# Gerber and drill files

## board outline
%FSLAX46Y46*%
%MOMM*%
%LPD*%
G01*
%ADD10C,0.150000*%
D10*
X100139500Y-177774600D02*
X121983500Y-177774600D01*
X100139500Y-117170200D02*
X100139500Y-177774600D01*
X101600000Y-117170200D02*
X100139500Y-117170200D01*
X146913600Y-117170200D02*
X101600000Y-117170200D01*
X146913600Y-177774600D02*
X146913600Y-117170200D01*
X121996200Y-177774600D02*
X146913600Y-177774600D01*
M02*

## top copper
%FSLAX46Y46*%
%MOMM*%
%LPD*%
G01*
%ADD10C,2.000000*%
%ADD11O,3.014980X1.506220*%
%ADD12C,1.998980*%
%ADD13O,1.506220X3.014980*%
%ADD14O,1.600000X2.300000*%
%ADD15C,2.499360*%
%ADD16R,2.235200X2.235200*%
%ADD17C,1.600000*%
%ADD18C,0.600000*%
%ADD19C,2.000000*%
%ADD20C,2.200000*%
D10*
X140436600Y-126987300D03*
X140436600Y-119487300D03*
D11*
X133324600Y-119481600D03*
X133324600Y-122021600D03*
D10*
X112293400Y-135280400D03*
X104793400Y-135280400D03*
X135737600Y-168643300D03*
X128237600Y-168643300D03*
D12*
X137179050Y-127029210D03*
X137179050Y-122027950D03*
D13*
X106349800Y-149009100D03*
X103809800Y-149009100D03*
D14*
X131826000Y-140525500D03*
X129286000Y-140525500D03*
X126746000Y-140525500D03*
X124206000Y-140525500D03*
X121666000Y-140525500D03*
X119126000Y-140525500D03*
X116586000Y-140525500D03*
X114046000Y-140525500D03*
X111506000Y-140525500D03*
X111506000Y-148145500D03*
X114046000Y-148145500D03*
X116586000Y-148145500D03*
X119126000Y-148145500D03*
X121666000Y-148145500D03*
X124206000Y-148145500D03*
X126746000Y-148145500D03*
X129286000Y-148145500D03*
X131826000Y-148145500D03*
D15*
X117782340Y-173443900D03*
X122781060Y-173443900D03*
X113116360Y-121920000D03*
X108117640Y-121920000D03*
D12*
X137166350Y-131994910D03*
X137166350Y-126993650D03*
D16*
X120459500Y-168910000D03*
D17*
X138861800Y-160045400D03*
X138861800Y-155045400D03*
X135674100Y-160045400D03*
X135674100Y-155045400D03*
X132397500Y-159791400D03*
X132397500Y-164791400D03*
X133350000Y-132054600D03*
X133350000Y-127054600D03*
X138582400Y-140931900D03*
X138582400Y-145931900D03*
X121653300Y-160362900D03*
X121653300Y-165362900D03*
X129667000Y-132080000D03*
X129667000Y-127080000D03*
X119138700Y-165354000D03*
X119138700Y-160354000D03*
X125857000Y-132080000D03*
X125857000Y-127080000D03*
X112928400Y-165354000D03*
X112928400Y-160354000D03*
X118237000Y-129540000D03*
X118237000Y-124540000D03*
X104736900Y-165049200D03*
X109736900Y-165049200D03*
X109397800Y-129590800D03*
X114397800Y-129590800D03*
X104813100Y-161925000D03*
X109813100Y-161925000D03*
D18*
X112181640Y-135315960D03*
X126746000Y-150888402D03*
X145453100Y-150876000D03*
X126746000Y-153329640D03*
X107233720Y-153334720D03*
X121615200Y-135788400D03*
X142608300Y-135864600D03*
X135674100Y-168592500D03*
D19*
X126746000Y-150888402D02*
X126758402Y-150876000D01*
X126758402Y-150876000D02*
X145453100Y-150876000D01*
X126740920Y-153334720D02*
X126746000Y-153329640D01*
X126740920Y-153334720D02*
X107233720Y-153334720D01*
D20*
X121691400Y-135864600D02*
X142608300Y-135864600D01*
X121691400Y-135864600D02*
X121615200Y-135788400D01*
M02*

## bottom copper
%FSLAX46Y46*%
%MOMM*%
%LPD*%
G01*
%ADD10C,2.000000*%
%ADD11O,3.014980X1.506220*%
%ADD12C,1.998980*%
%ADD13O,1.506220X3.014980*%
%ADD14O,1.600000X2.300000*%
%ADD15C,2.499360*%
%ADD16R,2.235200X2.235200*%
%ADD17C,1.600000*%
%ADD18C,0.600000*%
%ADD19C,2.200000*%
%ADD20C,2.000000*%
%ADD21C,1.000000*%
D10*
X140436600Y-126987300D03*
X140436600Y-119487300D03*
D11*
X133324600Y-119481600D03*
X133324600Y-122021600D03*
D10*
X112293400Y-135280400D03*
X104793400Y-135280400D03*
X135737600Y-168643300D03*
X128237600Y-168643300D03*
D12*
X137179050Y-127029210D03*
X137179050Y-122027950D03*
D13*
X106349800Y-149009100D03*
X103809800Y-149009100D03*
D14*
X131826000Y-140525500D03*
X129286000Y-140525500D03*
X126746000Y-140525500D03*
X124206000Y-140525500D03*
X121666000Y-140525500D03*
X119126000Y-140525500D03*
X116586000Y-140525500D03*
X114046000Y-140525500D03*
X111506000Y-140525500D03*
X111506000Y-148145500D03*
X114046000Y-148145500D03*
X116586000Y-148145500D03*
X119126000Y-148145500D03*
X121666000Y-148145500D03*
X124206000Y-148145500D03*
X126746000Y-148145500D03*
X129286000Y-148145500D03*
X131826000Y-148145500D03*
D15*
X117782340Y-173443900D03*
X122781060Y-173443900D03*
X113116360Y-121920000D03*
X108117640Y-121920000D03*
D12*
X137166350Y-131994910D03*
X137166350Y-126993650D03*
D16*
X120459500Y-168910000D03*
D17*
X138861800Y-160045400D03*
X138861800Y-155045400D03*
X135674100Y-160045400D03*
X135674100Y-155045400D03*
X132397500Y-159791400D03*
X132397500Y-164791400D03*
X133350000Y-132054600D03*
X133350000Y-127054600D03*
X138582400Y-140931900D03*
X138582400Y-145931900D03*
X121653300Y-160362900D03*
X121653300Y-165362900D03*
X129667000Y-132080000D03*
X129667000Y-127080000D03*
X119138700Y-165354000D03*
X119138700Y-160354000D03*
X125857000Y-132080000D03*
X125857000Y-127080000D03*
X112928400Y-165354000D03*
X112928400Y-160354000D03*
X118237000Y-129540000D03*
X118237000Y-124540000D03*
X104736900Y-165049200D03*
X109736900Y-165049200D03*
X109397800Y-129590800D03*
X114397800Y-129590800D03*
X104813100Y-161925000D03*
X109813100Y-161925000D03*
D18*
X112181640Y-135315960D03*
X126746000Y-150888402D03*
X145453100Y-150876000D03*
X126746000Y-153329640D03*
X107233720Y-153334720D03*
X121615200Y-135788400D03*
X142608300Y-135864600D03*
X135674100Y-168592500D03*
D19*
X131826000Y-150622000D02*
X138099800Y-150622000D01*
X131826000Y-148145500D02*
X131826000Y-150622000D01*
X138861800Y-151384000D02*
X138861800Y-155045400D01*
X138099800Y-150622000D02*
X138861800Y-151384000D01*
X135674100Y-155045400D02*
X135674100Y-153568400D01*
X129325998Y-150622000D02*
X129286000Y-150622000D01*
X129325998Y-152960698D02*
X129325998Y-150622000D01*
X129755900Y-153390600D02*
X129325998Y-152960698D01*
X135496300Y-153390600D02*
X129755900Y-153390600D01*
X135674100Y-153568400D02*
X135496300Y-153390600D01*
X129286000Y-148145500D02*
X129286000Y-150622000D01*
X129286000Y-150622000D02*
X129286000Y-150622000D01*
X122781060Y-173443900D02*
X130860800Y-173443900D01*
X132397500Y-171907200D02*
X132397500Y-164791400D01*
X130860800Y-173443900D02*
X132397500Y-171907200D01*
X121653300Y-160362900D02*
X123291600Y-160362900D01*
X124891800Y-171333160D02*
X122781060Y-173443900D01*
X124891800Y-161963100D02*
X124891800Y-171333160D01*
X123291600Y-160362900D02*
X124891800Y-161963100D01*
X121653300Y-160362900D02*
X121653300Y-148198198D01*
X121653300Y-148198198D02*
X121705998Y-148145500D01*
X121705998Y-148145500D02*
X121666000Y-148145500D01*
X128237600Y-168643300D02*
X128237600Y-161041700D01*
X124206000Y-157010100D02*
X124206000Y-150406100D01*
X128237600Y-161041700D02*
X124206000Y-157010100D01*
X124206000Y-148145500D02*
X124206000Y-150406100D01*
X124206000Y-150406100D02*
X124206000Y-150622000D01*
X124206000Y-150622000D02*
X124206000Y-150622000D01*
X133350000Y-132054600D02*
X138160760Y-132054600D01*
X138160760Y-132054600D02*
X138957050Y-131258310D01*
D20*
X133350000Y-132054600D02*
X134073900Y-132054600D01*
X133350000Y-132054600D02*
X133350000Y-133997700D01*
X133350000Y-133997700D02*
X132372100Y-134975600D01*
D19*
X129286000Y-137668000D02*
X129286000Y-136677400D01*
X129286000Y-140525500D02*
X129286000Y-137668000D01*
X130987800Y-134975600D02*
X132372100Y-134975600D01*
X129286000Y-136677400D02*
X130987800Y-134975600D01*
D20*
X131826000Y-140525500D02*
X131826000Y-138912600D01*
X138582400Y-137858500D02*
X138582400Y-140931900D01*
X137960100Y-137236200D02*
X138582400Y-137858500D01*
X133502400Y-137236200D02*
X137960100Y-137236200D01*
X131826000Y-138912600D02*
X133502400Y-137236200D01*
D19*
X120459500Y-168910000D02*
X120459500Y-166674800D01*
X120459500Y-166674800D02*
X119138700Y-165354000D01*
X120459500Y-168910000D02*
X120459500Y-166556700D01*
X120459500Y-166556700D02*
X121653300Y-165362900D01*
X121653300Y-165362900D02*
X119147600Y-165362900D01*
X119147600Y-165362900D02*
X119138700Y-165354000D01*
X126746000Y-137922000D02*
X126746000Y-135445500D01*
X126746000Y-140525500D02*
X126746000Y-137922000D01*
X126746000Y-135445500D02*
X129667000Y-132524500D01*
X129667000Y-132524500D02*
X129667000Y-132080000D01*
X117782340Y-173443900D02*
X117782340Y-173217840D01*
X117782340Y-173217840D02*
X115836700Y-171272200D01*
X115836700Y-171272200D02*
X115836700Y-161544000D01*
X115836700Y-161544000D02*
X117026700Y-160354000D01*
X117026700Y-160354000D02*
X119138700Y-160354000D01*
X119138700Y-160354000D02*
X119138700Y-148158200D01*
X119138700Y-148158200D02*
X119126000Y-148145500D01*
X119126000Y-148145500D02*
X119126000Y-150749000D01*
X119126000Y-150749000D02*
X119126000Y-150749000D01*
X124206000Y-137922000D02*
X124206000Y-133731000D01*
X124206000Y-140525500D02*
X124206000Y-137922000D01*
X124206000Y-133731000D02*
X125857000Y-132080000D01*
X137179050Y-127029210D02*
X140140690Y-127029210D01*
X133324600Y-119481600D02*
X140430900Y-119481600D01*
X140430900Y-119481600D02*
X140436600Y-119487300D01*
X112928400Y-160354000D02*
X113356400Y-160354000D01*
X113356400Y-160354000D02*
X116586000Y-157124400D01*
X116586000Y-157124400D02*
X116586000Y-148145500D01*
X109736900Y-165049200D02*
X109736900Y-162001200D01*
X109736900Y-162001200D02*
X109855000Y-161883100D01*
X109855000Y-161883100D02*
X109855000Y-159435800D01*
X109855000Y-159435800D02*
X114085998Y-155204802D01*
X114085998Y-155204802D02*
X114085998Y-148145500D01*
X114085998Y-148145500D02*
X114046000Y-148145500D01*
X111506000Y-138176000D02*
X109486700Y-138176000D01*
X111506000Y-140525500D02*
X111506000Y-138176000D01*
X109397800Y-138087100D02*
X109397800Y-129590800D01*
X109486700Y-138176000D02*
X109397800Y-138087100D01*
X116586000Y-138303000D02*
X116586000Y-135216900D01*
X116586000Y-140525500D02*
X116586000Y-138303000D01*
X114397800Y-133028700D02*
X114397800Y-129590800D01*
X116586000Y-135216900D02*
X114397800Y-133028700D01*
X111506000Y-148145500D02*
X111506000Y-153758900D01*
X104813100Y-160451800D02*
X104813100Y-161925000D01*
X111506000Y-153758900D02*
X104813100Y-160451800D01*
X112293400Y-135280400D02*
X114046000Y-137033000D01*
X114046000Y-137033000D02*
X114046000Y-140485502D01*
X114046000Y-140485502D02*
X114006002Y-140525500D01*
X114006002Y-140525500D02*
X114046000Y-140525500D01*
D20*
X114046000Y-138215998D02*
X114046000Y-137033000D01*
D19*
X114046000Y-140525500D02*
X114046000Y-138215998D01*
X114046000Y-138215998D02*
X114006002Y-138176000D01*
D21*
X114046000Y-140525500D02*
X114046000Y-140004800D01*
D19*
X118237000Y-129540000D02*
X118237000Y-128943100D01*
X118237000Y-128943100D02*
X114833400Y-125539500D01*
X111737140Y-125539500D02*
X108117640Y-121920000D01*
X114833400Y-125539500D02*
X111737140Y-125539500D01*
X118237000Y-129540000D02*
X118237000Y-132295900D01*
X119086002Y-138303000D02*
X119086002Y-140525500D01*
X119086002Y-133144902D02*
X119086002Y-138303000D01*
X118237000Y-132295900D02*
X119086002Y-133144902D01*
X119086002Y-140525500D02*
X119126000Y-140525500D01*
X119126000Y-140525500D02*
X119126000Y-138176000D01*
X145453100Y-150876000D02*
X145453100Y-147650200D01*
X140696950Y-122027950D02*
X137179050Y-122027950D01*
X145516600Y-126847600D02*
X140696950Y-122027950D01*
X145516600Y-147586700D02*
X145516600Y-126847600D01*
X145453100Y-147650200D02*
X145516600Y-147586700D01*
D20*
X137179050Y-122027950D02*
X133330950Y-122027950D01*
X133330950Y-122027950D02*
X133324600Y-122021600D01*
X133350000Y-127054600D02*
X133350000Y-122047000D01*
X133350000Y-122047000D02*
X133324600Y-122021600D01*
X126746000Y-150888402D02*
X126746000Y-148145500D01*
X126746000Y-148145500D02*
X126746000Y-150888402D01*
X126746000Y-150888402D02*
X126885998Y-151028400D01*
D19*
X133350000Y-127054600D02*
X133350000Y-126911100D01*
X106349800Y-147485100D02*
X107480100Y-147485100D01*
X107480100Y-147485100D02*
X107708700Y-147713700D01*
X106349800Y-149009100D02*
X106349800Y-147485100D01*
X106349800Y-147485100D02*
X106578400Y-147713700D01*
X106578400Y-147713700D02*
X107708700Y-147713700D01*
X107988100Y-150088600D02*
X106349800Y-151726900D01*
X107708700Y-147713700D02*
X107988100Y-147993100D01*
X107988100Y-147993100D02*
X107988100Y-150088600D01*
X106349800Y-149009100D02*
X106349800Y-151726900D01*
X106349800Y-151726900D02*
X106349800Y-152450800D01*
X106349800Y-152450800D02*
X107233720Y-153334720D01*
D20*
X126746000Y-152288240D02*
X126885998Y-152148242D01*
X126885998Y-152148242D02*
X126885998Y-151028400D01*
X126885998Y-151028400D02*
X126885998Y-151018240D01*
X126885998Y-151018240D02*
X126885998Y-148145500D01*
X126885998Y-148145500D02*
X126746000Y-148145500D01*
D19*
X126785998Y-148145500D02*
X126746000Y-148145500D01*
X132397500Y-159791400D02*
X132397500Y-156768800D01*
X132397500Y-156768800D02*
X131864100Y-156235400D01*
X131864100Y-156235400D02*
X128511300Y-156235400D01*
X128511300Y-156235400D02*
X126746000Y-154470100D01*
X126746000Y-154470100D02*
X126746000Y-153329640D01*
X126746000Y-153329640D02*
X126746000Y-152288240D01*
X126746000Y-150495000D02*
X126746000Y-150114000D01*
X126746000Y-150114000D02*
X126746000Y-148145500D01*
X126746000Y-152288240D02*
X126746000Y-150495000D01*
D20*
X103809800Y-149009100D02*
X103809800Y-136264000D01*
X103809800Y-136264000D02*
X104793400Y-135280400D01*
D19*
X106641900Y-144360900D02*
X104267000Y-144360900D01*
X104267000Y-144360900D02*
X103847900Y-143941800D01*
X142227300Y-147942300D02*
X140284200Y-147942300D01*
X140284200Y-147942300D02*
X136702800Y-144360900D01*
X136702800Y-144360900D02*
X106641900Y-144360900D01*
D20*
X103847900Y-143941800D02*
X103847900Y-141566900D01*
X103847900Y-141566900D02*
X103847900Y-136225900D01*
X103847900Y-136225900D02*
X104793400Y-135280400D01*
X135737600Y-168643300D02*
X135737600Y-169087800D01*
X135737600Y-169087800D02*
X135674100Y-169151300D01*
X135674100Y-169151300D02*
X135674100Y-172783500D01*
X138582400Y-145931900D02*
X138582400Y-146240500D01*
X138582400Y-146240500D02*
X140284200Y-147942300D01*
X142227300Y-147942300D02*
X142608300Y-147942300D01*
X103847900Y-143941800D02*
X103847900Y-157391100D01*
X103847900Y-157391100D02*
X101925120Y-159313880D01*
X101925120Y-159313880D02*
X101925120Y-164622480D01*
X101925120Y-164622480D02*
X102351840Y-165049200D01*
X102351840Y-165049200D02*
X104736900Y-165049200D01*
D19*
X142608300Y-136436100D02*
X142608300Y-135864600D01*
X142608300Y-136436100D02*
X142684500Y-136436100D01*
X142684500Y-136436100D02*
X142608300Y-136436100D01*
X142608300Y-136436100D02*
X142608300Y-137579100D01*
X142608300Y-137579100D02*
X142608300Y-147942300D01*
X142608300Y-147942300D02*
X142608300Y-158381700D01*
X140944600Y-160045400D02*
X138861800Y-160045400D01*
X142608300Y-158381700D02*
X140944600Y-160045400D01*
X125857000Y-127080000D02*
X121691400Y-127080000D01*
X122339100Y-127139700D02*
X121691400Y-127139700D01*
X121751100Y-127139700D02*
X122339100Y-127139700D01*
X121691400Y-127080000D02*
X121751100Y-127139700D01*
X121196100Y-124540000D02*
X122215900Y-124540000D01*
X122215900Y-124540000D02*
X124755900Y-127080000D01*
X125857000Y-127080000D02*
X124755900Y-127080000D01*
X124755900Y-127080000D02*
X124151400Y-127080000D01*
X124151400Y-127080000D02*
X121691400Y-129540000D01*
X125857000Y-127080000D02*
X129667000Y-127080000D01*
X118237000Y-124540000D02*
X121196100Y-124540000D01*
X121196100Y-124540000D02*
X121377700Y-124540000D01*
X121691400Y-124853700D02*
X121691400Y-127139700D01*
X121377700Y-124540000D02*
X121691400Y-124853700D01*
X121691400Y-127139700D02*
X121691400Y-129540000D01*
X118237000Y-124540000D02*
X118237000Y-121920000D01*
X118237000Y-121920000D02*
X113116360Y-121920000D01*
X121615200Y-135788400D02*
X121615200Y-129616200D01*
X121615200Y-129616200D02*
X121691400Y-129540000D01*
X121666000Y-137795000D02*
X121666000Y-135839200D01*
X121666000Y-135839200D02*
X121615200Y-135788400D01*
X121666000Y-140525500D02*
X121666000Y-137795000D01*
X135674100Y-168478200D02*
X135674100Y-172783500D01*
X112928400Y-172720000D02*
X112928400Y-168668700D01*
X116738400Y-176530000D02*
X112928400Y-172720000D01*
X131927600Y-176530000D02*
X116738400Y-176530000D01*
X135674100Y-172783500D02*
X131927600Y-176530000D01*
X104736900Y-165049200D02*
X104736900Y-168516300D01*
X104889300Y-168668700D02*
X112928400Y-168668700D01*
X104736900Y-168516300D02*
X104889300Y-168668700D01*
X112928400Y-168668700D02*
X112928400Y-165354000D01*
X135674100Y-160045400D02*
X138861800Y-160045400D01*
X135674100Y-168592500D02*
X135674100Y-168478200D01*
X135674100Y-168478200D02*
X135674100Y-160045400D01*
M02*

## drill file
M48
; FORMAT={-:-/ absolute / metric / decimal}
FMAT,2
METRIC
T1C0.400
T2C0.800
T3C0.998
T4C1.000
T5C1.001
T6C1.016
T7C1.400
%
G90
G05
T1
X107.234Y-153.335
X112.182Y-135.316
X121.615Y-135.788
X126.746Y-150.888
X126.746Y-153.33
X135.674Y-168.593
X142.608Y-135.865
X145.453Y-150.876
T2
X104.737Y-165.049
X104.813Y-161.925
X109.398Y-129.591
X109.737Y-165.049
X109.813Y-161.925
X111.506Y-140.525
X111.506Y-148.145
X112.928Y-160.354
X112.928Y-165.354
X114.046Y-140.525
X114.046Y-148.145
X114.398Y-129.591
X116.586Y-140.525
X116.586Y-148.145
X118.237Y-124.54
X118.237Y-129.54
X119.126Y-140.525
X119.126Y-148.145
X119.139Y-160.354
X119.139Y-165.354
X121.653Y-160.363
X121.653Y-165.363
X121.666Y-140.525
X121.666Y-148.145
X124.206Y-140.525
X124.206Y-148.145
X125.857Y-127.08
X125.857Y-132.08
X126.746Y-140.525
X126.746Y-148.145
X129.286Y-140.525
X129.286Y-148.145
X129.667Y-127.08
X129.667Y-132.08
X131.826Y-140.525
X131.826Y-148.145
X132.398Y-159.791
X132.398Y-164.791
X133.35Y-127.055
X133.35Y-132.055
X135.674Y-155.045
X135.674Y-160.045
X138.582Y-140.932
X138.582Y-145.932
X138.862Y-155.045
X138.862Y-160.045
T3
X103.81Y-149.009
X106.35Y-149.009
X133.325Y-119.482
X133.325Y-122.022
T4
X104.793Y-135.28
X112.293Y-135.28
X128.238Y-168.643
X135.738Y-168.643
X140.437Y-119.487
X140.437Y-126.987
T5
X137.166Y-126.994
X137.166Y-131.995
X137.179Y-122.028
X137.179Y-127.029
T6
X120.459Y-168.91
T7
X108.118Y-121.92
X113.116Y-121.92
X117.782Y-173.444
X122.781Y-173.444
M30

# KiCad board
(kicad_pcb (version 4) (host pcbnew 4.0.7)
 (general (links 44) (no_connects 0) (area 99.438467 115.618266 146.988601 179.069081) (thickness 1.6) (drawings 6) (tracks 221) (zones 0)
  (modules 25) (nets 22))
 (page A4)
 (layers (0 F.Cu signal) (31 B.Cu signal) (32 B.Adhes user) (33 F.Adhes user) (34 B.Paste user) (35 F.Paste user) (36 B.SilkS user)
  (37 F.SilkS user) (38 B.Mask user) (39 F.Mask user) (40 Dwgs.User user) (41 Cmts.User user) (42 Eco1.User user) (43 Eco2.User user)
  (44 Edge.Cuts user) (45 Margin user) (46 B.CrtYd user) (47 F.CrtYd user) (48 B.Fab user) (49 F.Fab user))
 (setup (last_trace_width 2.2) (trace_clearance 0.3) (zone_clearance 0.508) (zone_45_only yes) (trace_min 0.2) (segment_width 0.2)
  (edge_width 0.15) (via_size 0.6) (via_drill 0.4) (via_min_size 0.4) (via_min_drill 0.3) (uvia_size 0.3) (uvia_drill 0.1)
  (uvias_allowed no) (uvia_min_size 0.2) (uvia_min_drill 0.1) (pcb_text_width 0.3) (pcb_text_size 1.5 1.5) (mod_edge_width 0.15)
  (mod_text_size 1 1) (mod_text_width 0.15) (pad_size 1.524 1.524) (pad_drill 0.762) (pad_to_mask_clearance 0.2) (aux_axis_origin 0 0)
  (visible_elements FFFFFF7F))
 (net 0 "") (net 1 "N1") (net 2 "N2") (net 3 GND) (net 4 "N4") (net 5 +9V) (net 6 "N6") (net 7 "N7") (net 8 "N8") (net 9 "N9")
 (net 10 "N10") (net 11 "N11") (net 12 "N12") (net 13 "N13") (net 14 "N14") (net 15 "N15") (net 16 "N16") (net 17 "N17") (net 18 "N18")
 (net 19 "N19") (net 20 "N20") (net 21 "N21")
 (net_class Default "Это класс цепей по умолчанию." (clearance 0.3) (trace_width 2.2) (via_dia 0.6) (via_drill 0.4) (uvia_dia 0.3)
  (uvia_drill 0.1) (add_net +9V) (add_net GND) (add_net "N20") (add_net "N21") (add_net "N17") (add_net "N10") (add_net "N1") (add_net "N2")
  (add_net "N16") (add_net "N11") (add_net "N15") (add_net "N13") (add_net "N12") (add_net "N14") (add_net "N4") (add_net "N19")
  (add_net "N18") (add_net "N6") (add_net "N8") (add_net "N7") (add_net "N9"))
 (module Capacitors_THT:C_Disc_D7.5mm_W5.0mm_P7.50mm (layer F.Cu) (at 140.4366 126.9873 90)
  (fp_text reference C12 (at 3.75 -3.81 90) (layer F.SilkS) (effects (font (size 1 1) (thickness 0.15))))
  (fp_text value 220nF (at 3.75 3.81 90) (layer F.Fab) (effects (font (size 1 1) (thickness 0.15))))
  (pad 1 thru_hole circle (at 0 0 90) (size 2 2) (drill 1) (layers *.Cu *.Mask) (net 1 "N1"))
  (pad 2 thru_hole circle (at 7.5 0 90) (size 2 2) (drill 1) (layers *.Cu *.Mask) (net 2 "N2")))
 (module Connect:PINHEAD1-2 (layer F.Cu) (at 133.3246 120.7516 270)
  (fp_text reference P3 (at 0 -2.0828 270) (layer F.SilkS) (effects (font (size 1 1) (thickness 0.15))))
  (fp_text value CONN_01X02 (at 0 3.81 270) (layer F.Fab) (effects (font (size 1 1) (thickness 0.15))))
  (pad 1 thru_hole oval (at -1.27 0 270) (size 1.50622 3.01498) (drill 0.99822) (layers *.Cu *.Mask) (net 2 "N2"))
  (pad 2 thru_hole oval (at 1.27 0 270) (size 1.50622 3.01498) (drill 0.99822) (layers *.Cu *.Mask) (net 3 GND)))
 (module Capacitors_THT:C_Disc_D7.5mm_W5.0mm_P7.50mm (layer F.Cu) (at 112.2934 135.2804 180)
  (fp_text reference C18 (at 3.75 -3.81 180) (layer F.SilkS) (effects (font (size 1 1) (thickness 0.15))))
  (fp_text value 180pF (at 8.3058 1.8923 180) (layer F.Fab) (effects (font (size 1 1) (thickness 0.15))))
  (pad 1 thru_hole circle (at 0 0 180) (size 2 2) (drill 1) (layers *.Cu *.Mask) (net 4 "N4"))
  (pad 2 thru_hole circle (at 7.5 0 180) (size 2 2) (drill 1) (layers *.Cu *.Mask) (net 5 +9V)))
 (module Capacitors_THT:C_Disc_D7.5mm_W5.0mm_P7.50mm (layer F.Cu) (at 135.7376 168.6433 180)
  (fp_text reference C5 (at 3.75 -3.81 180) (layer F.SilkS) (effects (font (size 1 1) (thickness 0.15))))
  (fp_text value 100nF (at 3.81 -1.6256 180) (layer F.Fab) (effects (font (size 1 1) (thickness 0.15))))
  (pad 1 thru_hole circle (at 0 0 180) (size 2 2) (drill 1) (layers *.Cu *.Mask) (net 5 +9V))
  (pad 2 thru_hole circle (at 7.5 0 180) (size 2 2) (drill 1) (layers *.Cu *.Mask) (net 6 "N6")))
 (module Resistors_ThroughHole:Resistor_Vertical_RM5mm (layer F.Cu) (at 137.17905 124.52985 90)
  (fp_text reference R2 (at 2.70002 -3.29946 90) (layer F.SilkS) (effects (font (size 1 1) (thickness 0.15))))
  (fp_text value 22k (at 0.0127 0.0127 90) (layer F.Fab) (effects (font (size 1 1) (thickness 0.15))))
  (pad 1 thru_hole circle (at -2.49936 0 90) (size 1.99898 1.99898) (drill 1.00076) (layers *.Cu *.SilkS *.Mask) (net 1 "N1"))
  (pad 2 thru_hole circle (at 2.5019 0 90) (size 1.99898 1.99898) (drill 1.00076) (layers *.Cu *.SilkS *.Mask) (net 3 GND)))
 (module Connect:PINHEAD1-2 (layer F.Cu) (at 105.0798 149.0091 180)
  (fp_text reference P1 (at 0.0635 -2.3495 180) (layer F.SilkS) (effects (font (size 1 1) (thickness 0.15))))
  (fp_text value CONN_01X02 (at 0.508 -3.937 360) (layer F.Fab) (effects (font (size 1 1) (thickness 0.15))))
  (pad 1 thru_hole oval (at -1.27 0 180) (size 1.50622 3.01498) (drill 0.99822) (layers *.Cu *.Mask) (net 3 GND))
  (pad 2 thru_hole oval (at 1.27 0 180) (size 1.50622 3.01498) (drill 0.99822) (layers *.Cu *.Mask) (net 5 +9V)))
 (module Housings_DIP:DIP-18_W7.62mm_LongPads (layer F.Cu) (at 131.826 140.5255 270)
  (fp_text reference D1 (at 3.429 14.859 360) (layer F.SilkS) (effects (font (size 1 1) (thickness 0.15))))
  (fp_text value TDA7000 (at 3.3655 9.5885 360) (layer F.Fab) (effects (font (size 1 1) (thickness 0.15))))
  (pad 1 thru_hole oval (at 0 0 270) (size 2.3 1.6) (drill 0.8) (layers *.Cu *.Mask F.SilkS) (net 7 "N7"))
  (pad 2 thru_hole oval (at 0 2.54 270) (size 2.3 1.6) (drill 0.8) (layers *.Cu *.Mask F.SilkS) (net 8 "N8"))
  (pad 3 thru_hole oval (at 0 5.08 270) (size 2.3 1.6) (drill 0.8) (layers *.Cu *.Mask F.SilkS) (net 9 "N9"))
  (pad 4 thru_hole oval (at 0 7.62 270) (size 2.3 1.6) (drill 0.8) (layers *.Cu *.Mask F.SilkS) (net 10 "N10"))
  (pad 5 thru_hole oval (at 0 10.16 270) (size 2.3 1.6) (drill 0.8) (layers *.Cu *.Mask F.SilkS) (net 5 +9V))
  (pad 6 thru_hole oval (at 0 12.7 270) (size 2.3 1.6) (drill 0.8) (layers *.Cu *.Mask F.SilkS) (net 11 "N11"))
  (pad 7 thru_hole oval (at 0 15.24 270) (size 2.3 1.6) (drill 0.8) (layers *.Cu *.Mask F.SilkS) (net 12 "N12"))
  (pad 8 thru_hole oval (at 0 17.78 270) (size 2.3 1.6) (drill 0.8) (layers *.Cu *.Mask F.SilkS) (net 4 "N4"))
  (pad 9 thru_hole oval (at 0 20.32 270) (size 2.3 1.6) (drill 0.8) (layers *.Cu *.Mask F.SilkS) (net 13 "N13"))
  (pad 10 thru_hole oval (at 7.62 20.32 270) (size 2.3 1.6) (drill 0.8) (layers *.Cu *.Mask F.SilkS) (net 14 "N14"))
  (pad 11 thru_hole oval (at 7.62 17.78 270) (size 2.3 1.6) (drill 0.8) (layers *.Cu *.Mask F.SilkS) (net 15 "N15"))
  (pad 12 thru_hole oval (at 7.62 15.24 270) (size 2.3 1.6) (drill 0.8) (layers *.Cu *.Mask F.SilkS) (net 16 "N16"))
  (pad 13 thru_hole oval (at 7.62 12.7 270) (size 2.3 1.6) (drill 0.8) (layers *.Cu *.Mask F.SilkS) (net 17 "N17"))
  (pad 14 thru_hole oval (at 7.62 10.16 270) (size 2.3 1.6) (drill 0.8) (layers *.Cu *.Mask F.SilkS) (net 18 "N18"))
  (pad 15 thru_hole oval (at 7.62 7.62 270) (size 2.3 1.6) (drill 0.8) (layers *.Cu *.Mask F.SilkS) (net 6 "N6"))
  (pad 16 thru_hole oval (at 7.62 5.08 270) (size 2.3 1.6) (drill 0.8) (layers *.Cu *.Mask F.SilkS) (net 3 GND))
  (pad 17 thru_hole oval (at 7.62 2.54 270) (size 2.3 1.6) (drill 0.8) (layers *.Cu *.Mask F.SilkS) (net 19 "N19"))
  (pad 18 thru_hole oval (at 7.62 0 270) (size 2.3 1.6) (drill 0.8) (layers *.Cu *.Mask F.SilkS) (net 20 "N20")))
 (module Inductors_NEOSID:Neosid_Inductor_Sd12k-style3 (layer F.Cu) (at 120.2817 173.4439 180)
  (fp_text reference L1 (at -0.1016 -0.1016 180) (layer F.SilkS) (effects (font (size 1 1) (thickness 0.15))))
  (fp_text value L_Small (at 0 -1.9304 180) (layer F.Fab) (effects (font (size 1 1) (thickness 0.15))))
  (pad 2 thru_hole circle (at 2.49936 0 180) (size 2.49936 2.49936) (drill 1.39954) (layers *.Cu *.Mask F.SilkS) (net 17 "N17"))
  (pad 1 thru_hole circle (at -2.49936 0 180) (size 2.49936 2.49936) (drill 1.39954) (layers *.Cu *.Mask F.SilkS) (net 18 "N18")))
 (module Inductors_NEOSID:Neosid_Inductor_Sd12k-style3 (layer F.Cu) (at 110.617 121.92)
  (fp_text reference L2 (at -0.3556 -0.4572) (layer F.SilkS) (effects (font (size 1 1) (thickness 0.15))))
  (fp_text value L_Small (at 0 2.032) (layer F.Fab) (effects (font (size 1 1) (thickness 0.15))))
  (pad 2 thru_hole circle (at 2.49936 0) (size 2.49936 2.49936) (drill 1.39954) (layers *.Cu *.Mask F.SilkS) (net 5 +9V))
  (pad 1 thru_hole circle (at -2.49936 0) (size 2.49936 2.49936) (drill 1.39954) (layers *.Cu *.Mask F.SilkS) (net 11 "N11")))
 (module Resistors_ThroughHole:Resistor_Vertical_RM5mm (layer F.Cu) (at 137.16635 129.49555 90)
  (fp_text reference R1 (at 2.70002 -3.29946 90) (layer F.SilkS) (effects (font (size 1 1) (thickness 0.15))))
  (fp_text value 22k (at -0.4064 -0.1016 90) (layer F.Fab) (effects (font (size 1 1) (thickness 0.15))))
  (pad 1 thru_hole circle (at -2.49936 0 90) (size 1.99898 1.99898) (drill 1.00076) (layers *.Cu *.SilkS *.Mask) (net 8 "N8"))
  (pad 2 thru_hole circle (at 2.5019 0 90) (size 1.99898 1.99898) (drill 1.00076) (layers *.Cu *.SilkS *.Mask) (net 1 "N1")))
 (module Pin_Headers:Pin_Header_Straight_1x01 (layer F.Cu) (at 120.4595 168.91)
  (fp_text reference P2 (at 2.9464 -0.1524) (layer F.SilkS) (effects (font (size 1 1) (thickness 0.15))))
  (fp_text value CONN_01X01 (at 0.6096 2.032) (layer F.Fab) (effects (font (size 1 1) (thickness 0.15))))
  (pad 1 thru_hole rect (at 0 0) (size 2.2352 2.2352) (drill 1.016) (layers *.Cu *.Mask F.SilkS) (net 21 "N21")))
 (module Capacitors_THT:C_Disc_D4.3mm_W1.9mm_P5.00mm (layer F.Cu) (at 138.8618 160.0454 90)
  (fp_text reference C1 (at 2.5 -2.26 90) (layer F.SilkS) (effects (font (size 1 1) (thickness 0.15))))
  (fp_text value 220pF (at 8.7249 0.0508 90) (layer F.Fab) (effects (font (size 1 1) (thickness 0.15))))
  (pad 1 thru_hole circle (at 0 0 90) (size 1.6 1.6) (drill 0.8) (layers *.Cu *.Mask) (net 5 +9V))
  (pad 2 thru_hole circle (at 5 0 90) (size 1.6 1.6) (drill 0.8) (layers *.Cu *.Mask) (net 20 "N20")))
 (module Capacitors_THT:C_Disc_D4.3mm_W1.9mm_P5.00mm (layer F.Cu) (at 135.6741 160.0454 90)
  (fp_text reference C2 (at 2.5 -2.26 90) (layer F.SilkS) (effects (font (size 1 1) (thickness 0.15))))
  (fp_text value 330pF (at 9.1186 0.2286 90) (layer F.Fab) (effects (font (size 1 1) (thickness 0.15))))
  (pad 1 thru_hole circle (at 0 0 90) (size 1.6 1.6) (drill 0.8) (layers *.Cu *.Mask) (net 5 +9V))
  (pad 2 thru_hole circle (at 5 0 90) (size 1.6 1.6) (drill 0.8) (layers *.Cu *.Mask) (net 19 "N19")))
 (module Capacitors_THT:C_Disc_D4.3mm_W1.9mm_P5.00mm (layer F.Cu) (at 132.3975 159.7914 270)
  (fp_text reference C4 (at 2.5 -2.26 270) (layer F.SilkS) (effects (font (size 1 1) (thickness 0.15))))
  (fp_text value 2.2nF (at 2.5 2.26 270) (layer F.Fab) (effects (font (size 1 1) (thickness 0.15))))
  (pad 1 thru_hole circle (at 0 0 270) (size 1.6 1.6) (drill 0.8) (layers *.Cu *.Mask) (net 3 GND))
  (pad 2 thru_hole circle (at 5 0 270) (size 1.6 1.6) (drill 0.8) (layers *.Cu *.Mask) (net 18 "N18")))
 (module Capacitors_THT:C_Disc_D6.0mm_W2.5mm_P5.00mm (layer F.Cu) (at 133.35 132.0546 90)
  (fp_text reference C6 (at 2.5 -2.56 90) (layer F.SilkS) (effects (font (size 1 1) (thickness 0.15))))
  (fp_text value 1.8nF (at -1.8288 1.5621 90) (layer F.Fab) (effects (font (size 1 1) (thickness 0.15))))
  (pad 1 thru_hole circle (at 0 0 90) (size 1.6 1.6) (drill 0.8) (layers *.Cu *.Mask) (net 8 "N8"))
  (pad 2 thru_hole circle (at 5 0 90) (size 1.6 1.6) (drill 0.8) (layers *.Cu *.Mask) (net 3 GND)))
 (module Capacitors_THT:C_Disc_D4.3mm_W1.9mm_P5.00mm (layer F.Cu) (at 138.5824 140.9319 270)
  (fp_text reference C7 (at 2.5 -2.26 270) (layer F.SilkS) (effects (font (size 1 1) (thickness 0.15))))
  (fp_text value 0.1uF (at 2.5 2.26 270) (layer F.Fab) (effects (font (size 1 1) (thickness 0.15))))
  (pad 1 thru_hole circle (at 0 0 270) (size 1.6 1.6) (drill 0.8) (layers *.Cu *.Mask) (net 7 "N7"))
  (pad 2 thru_hole circle (at 5 0 270) (size 1.6 1.6) (drill 0.8) (layers *.Cu *.Mask) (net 5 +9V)))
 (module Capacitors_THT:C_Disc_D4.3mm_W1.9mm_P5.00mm (layer F.Cu) (at 121.6533 160.3629 270)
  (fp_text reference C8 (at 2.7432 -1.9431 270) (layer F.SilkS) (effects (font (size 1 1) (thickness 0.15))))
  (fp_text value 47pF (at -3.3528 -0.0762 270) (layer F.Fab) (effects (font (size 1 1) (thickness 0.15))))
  (pad 1 thru_hole circle (at 0 0 270) (size 1.6 1.6) (drill 0.8) (layers *.Cu *.Mask) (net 18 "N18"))
  (pad 2 thru_hole circle (at 5 0 270) (size 1.6 1.6) (drill 0.8) (layers *.Cu *.Mask) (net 21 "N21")))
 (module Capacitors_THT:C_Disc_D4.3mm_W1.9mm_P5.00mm (layer F.Cu) (at 129.667 132.08 90)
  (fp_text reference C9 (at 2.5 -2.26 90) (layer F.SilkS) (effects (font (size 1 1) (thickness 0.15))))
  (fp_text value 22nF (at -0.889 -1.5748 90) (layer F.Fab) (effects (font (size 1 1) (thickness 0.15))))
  (pad 1 thru_hole circle (at 0 0 90) (size 1.6 1.6) (drill 0.8) (layers *.Cu *.Mask) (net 9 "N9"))
  (pad 2 thru_hole circle (at 5 0 90) (size 1.6 1.6) (drill 0.8) (layers *.Cu *.Mask) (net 5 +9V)))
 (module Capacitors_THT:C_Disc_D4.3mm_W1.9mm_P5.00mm (layer F.Cu) (at 119.1387 165.354 90)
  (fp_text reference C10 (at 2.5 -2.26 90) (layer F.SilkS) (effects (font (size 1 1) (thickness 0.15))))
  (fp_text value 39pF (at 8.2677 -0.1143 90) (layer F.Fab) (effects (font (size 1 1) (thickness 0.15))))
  (pad 1 thru_hole circle (at 0 0 90) (size 1.6 1.6) (drill 0.8) (layers *.Cu *.Mask) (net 21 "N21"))
  (pad 2 thru_hole circle (at 5 0 90) (size 1.6 1.6) (drill 0.8) (layers *.Cu *.Mask) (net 17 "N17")))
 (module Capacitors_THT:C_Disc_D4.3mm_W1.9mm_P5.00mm (layer F.Cu) (at 125.857 132.08 90)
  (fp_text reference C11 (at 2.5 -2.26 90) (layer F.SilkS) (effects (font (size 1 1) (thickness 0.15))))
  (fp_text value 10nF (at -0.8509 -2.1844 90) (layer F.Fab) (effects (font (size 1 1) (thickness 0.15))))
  (pad 1 thru_hole circle (at 0 0 90) (size 1.6 1.6) (drill 0.8) (layers *.Cu *.Mask) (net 10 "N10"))
  (pad 2 thru_hole circle (at 5 0 90) (size 1.6 1.6) (drill 0.8) (layers *.Cu *.Mask) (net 5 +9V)))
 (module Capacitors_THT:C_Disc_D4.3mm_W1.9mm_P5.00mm (layer F.Cu) (at 112.9284 165.354 90)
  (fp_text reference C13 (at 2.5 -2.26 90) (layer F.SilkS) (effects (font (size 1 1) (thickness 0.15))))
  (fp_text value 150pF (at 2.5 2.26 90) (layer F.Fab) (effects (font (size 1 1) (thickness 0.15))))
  (pad 1 thru_hole circle (at 0 0 90) (size 1.6 1.6) (drill 0.8) (layers *.Cu *.Mask) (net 5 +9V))
  (pad 2 thru_hole circle (at 5 0 90) (size 1.6 1.6) (drill 0.8) (layers *.Cu *.Mask) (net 16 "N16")))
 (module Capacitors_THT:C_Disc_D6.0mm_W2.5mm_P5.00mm (layer F.Cu) (at 118.237 129.54 90)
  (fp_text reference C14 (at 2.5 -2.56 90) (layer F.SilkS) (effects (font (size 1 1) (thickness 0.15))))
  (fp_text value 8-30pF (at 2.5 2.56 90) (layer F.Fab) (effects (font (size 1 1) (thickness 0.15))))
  (pad 1 thru_hole circle (at 0 0 90) (size 1.6 1.6) (drill 0.8) (layers *.Cu *.Mask) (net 11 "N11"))
  (pad 2 thru_hole circle (at 5 0 90) (size 1.6 1.6) (drill 0.8) (layers *.Cu *.Mask) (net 5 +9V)))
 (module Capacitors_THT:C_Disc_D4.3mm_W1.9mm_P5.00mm (layer F.Cu) (at 104.7369 165.0492)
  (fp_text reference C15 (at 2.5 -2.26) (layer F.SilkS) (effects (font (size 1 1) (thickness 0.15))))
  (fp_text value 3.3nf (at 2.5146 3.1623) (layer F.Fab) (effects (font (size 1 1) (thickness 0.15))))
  (pad 1 thru_hole circle (at 0 0) (size 1.6 1.6) (drill 0.8) (layers *.Cu *.Mask) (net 5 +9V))
  (pad 2 thru_hole circle (at 5 0) (size 1.6 1.6) (drill 0.8) (layers *.Cu *.Mask) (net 15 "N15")))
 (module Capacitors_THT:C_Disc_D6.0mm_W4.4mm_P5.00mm (layer F.Cu) (at 109.3978 129.5908)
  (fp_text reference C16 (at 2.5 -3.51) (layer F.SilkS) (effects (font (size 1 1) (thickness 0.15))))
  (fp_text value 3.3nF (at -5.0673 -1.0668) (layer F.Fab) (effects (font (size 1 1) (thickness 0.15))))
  (pad 1 thru_hole circle (at 0 0) (size 1.6 1.6) (drill 0.8) (layers *.Cu *.Mask) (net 13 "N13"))
  (pad 2 thru_hole circle (at 5 0) (size 1.6 1.6) (drill 0.8) (layers *.Cu *.Mask) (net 12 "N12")))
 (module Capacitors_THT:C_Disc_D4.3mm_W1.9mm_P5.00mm (layer F.Cu) (at 104.8131 161.925)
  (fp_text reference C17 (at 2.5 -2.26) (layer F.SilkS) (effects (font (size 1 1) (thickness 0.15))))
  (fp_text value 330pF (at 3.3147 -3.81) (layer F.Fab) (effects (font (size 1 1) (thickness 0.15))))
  (pad 1 thru_hole circle (at 0 0) (size 1.6 1.6) (drill 0.8) (layers *.Cu *.Mask) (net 14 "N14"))
  (pad 2 thru_hole circle (at 5 0) (size 1.6 1.6) (drill 0.8) (layers *.Cu *.Mask) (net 15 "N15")))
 (gr_line (start 100.1395 177.7746) (end 121.9835 177.7746) (angle 90) (layer Edge.Cuts) (width 0.15))
 (gr_line (start 100.1395 117.1702) (end 100.1395 177.7746) (angle 90) (layer Edge.Cuts) (width 0.15))
 (gr_line (start 101.6 117.1702) (end 100.1395 117.1702) (angle 90) (layer Edge.Cuts) (width 0.15))
 (gr_line (start 146.9136 117.1702) (end 101.6 117.1702) (angle 90) (layer Edge.Cuts) (width 0.15))
 (gr_line (start 146.9136 177.7746) (end 146.9136 117.1702) (angle 90) (layer Edge.Cuts) (width 0.15))
 (gr_line (start 121.9962 177.7746) (end 146.9136 177.7746) (angle 90) (layer Edge.Cuts) (width 0.15))
 (segment (start 131.826 150.622) (end 138.0998 150.622) (width 2.2) (layer B.Cu) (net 20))
 (segment (start 131.826 148.1455) (end 131.826 150.622) (width 2.2) (layer B.Cu) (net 20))
 (segment (start 138.8618 151.384) (end 138.8618 155.0454) (width 2.2) (layer B.Cu) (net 20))
 (segment (start 138.0998 150.622) (end 138.8618 151.384) (width 2.2) (layer B.Cu) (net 20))
 (segment (start 135.6741 155.0454) (end 135.6741 153.5684) (width 2.2) (layer B.Cu) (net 19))
 (segment (start 129.325998 150.622) (end 129.286 150.622) (width 2.2) (layer B.Cu) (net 19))
 (segment (start 129.325998 152.960698) (end 129.325998 150.622) (width 2.2) (layer B.Cu) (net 19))
 (segment (start 129.7559 153.3906) (end 129.325998 152.960698) (width 2.2) (layer B.Cu) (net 19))
 (segment (start 135.4963 153.3906) (end 129.7559 153.3906) (width 2.2) (layer B.Cu) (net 19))
 (segment (start 135.6741 153.5684) (end 135.4963 153.3906) (width 2.2) (layer B.Cu) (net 19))
 (segment (start 129.286 148.1455) (end 129.286 150.622) (width 2.2) (layer B.Cu) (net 19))
 (segment (start 129.286 150.622) (end 129.286 150.622) (width 2.2) (layer B.Cu) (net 19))
 (segment (start 122.78106 173.4439) (end 130.8608 173.4439) (width 2.2) (layer B.Cu) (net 18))
 (segment (start 132.3975 171.9072) (end 132.3975 164.7914) (width 2.2) (layer B.Cu) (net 18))
 (segment (start 130.8608 173.4439) (end 132.3975 171.9072) (width 2.2) (layer B.Cu) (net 18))
 (segment (start 121.6533 160.3629) (end 123.2916 160.3629) (width 2.2) (layer B.Cu) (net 18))
 (segment (start 124.8918 171.33316) (end 122.78106 173.4439) (width 2.2) (layer B.Cu) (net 18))
 (segment (start 124.8918 161.9631) (end 124.8918 171.33316) (width 2.2) (layer B.Cu) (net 18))
 (segment (start 123.2916 160.3629) (end 124.8918 161.9631) (width 2.2) (layer B.Cu) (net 18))
 (segment (start 121.6533 160.3629) (end 121.6533 148.198198) (width 2.2) (layer B.Cu) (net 18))
 (segment (start 121.6533 148.198198) (end 121.705998 148.1455) (width 2.2) (layer B.Cu) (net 18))
 (segment (start 121.705998 148.1455) (end 121.666 148.1455) (width 2.2) (layer B.Cu) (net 18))
 (segment (start 128.2376 168.6433) (end 128.2376 161.0417) (width 2.2) (layer B.Cu) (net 6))
 (segment (start 124.206 157.0101) (end 124.206 150.4061) (width 2.2) (layer B.Cu) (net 6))
 (segment (start 128.2376 161.0417) (end 124.206 157.0101) (width 2.2) (layer B.Cu) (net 6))
 (segment (start 124.206 148.1455) (end 124.206 150.4061) (width 2.2) (layer B.Cu) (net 6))
 (segment (start 124.206 150.4061) (end 124.206 150.622) (width 2.2) (layer B.Cu) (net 6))
 (segment (start 124.206 150.622) (end 124.206 150.622) (width 2.2) (layer B.Cu) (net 6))
 (segment (start 133.35 132.0546) (end 138.16076 132.0546) (width 2.2) (layer B.Cu) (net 8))
 (segment (start 138.16076 132.0546) (end 138.95705 131.25831) (width 2.2) (layer B.Cu) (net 8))
 (segment (start 133.35 132.0546) (end 134.0739 132.0546) (width 2) (layer B.Cu) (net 8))
 (segment (start 133.35 132.0546) (end 133.35 133.9977) (width 2) (layer B.Cu) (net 8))
 (segment (start 133.35 133.9977) (end 132.3721 134.9756) (width 2) (layer B.Cu) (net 8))
 (segment (start 129.286 137.668) (end 129.286 136.6774) (width 2.2) (layer B.Cu) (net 8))
 (segment (start 129.286 140.5255) (end 129.286 137.668) (width 2.2) (layer B.Cu) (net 8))
 (segment (start 130.9878 134.9756) (end 132.3721 134.9756) (width 2.2) (layer B.Cu) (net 8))
 (segment (start 129.286 136.6774) (end 130.9878 134.9756) (width 2.2) (layer B.Cu) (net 8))
 (segment (start 131.826 140.5255) (end 131.826 138.9126) (width 2) (layer B.Cu) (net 7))
 (segment (start 138.5824 137.8585) (end 138.5824 140.9319) (width 2) (layer B.Cu) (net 7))
 (segment (start 137.9601 137.2362) (end 138.5824 137.8585) (width 2) (layer B.Cu) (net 7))
 (segment (start 133.5024 137.2362) (end 137.9601 137.2362) (width 2) (layer B.Cu) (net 7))
 (segment (start 131.826 138.9126) (end 133.5024 137.2362) (width 2) (layer B.Cu) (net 7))
 (segment (start 120.4595 168.91) (end 120.4595 166.6748) (width 2.2) (layer B.Cu) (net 21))
 (segment (start 120.4595 166.6748) (end 119.1387 165.354) (width 2.2) (layer B.Cu) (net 21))
 (segment (start 120.4595 168.91) (end 120.4595 166.5567) (width 2.2) (layer B.Cu) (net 21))
 (segment (start 120.4595 166.5567) (end 121.6533 165.3629) (width 2.2) (layer B.Cu) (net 21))
 (segment (start 121.6533 165.3629) (end 119.1476 165.3629) (width 2.2) (layer B.Cu) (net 21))
 (segment (start 119.1476 165.3629) (end 119.1387 165.354) (width 2.2) (layer B.Cu) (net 21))
 (segment (start 126.746 137.922) (end 126.746 135.4455) (width 2.2) (layer B.Cu) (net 9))
 (segment (start 126.746 140.5255) (end 126.746 137.922) (width 2.2) (layer B.Cu) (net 9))
 (segment (start 126.746 135.4455) (end 129.667 132.5245) (width 2.2) (layer B.Cu) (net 9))
 (segment (start 129.667 132.5245) (end 129.667 132.08) (width 2.2) (layer B.Cu) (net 9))
 (segment (start 117.78234 173.4439) (end 117.78234 173.21784) (width 2.2) (layer B.Cu) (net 17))
 (segment (start 117.78234 173.21784) (end 115.8367 171.2722) (width 2.2) (layer B.Cu) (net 17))
 (segment (start 115.8367 171.2722) (end 115.8367 161.544) (width 2.2) (layer B.Cu) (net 17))
 (segment (start 115.8367 161.544) (end 117.0267 160.354) (width 2.2) (layer B.Cu) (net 17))
 (segment (start 117.0267 160.354) (end 119.1387 160.354) (width 2.2) (layer B.Cu) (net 17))
 (segment (start 119.1387 160.354) (end 119.1387 148.1582) (width 2.2) (layer B.Cu) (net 17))
 (segment (start 119.1387 148.1582) (end 119.126 148.1455) (width 2.2) (layer B.Cu) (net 17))
 (segment (start 119.126 148.1455) (end 119.126 150.749) (width 2.2) (layer B.Cu) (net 17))
 (segment (start 119.126 150.749) (end 119.126 150.749) (width 2.2) (layer B.Cu) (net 17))
 (segment (start 124.206 137.922) (end 124.206 133.731) (width 2.2) (layer B.Cu) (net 10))
 (segment (start 124.206 140.5255) (end 124.206 137.922) (width 2.2) (layer B.Cu) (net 10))
 (segment (start 124.206 133.731) (end 125.857 132.08) (width 2.2) (layer B.Cu) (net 10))
 (segment (start 137.17905 127.02921) (end 140.14069 127.02921) (width 2.2) (layer B.Cu) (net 1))
 (segment (start 133.3246 119.4816) (end 140.4309 119.4816) (width 2.2) (layer B.Cu) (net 2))
 (segment (start 140.4309 119.4816) (end 140.4366 119.4873) (width 2.2) (layer B.Cu) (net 2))
 (segment (start 112.9284 160.354) (end 113.3564 160.354) (width 2.2) (layer B.Cu) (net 16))
 (segment (start 113.3564 160.354) (end 116.586 157.1244) (width 2.2) (layer B.Cu) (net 16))
 (segment (start 116.586 157.1244) (end 116.586 148.1455) (width 2.2) (layer B.Cu) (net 16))
 (segment (start 109.7369 165.0492) (end 109.7369 162.0012) (width 2.2) (layer B.Cu) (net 15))
 (segment (start 109.7369 162.0012) (end 109.855 161.8831) (width 2.2) (layer B.Cu) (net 15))
 (segment (start 109.855 161.8831) (end 109.855 159.4358) (width 2.2) (layer B.Cu) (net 15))
 (segment (start 109.855 159.4358) (end 114.085998 155.204802) (width 2.2) (layer B.Cu) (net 15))
 (segment (start 114.085998 155.204802) (end 114.085998 148.1455) (width 2.2) (layer B.Cu) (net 15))
 (segment (start 114.085998 148.1455) (end 114.046 148.1455) (width 2.2) (layer B.Cu) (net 15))
 (segment (start 111.506 138.176) (end 109.4867 138.176) (width 2.2) (layer B.Cu) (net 13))
 (segment (start 111.506 140.5255) (end 111.506 138.176) (width 2.2) (layer B.Cu) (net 13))
 (segment (start 109.3978 138.0871) (end 109.3978 129.5908) (width 2.2) (layer B.Cu) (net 13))
 (segment (start 109.4867 138.176) (end 109.3978 138.0871) (width 2.2) (layer B.Cu) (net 13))
 (segment (start 116.586 138.303) (end 116.586 135.2169) (width 2.2) (layer B.Cu) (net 12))
 (segment (start 116.586 140.5255) (end 116.586 138.303) (width 2.2) (layer B.Cu) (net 12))
 (segment (start 114.3978 133.0287) (end 114.3978 129.5908) (width 2.2) (layer B.Cu) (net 12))
 (segment (start 116.586 135.2169) (end 114.3978 133.0287) (width 2.2) (layer B.Cu) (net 12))
 (segment (start 111.506 148.1455) (end 111.506 153.7589) (width 2.2) (layer B.Cu) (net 14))
 (segment (start 104.8131 160.4518) (end 104.8131 161.925) (width 2.2) (layer B.Cu) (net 14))
 (segment (start 111.506 153.7589) (end 104.8131 160.4518) (width 2.2) (layer B.Cu) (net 14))
 (segment (start 112.2934 135.2804) (end 114.046 137.033) (width 2.2) (layer B.Cu) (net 4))
 (segment (start 114.046 137.033) (end 114.046 140.485502) (width 2.2) (layer B.Cu) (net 4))
 (segment (start 114.046 140.485502) (end 114.006002 140.5255) (width 2.2) (layer B.Cu) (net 4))
 (segment (start 114.006002 140.5255) (end 114.046 140.5255) (width 2.2) (layer B.Cu) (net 4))
 (segment (start 114.046 138.215998) (end 114.046 137.033) (width 2) (layer B.Cu) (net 4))
 (via (at 112.18164 135.31596) (size 0.6) (drill 0.4) (layers F.Cu B.Cu) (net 4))
 (segment (start 114.046 140.5255) (end 114.046 138.215998) (width 2.2) (layer B.Cu) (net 4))
 (segment (start 114.046 138.215998) (end 114.006002 138.176) (width 2.2) (layer B.Cu) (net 4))
 (segment (start 114.046 140.5255) (end 114.046 140.0048) (width 1) (layer B.Cu) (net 4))
 (segment (start 118.237 129.54) (end 118.237 128.9431) (width 2.2) (layer B.Cu) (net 11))
 (segment (start 118.237 128.9431) (end 114.8334 125.5395) (width 2.2) (layer B.Cu) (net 11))
 (segment (start 111.73714 125.5395) (end 108.11764 121.92) (width 2.2) (layer B.Cu) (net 11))
 (segment (start 114.8334 125.5395) (end 111.73714 125.5395) (width 2.2) (layer B.Cu) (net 11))
 (segment (start 118.237 129.54) (end 118.237 132.2959) (width 2.2) (layer B.Cu) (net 11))
 (segment (start 119.086002 138.303) (end 119.086002 140.5255) (width 2.2) (layer B.Cu) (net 11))
 (segment (start 119.086002 133.144902) (end 119.086002 138.303) (width 2.2) (layer B.Cu) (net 11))
 (segment (start 118.237 132.2959) (end 119.086002 133.144902) (width 2.2) (layer B.Cu) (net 11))
 (segment (start 119.086002 140.5255) (end 119.126 140.5255) (width 2.2) (layer B.Cu) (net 11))
 (segment (start 119.126 140.5255) (end 119.126 138.176) (width 2.2) (layer B.Cu) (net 11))
 (segment (start 145.4531 150.876) (end 145.4531 147.6502) (width 2.2) (layer B.Cu) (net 3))
 (segment (start 140.69695 122.02795) (end 137.17905 122.02795) (width 2.2) (layer B.Cu) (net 3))
 (segment (start 145.5166 126.8476) (end 140.69695 122.02795) (width 2.2) (layer B.Cu) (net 3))
 (segment (start 145.5166 147.5867) (end 145.5166 126.8476) (width 2.2) (layer B.Cu) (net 3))
 (segment (start 145.4531 147.6502) (end 145.5166 147.5867) (width 2.2) (layer B.Cu) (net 3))
 (segment (start 137.17905 122.02795) (end 133.33095 122.02795) (width 2) (layer B.Cu) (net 3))
 (segment (start 133.33095 122.02795) (end 133.3246 122.0216) (width 2) (layer B.Cu) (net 3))
 (segment (start 133.35 127.0546) (end 133.35 122.047) (width 2) (layer B.Cu) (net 3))
 (segment (start 133.35 122.047) (end 133.3246 122.0216) (width 2) (layer B.Cu) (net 3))
 (segment (start 126.746 150.888402) (end 126.746 148.1455) (width 2) (layer B.Cu) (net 3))
 (via (at 126.746 150.888402) (size 0.6) (drill 0.4) (layers F.Cu B.Cu) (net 3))
 (segment (start 126.746 150.888402) (end 126.758402 150.876) (width 2) (layer F.Cu) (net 3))
 (segment (start 126.758402 150.876) (end 145.4531 150.876) (width 2) (layer F.Cu) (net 3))
 (via (at 145.4531 150.876) (size 0.6) (drill 0.4) (layers F.Cu B.Cu) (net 3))
 (segment (start 126.746 148.1455) (end 126.746 150.888402) (width 2) (layer B.Cu) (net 3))
 (segment (start 126.746 150.888402) (end 126.885998 151.0284) (width 2) (layer B.Cu) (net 3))
 (segment (start 133.35 127.0546) (end 133.35 126.9111) (width 2.2) (layer B.Cu) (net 3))
 (segment (start 106.3498 147.4851) (end 107.4801 147.4851) (width 2.2) (layer B.Cu) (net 3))
 (segment (start 107.4801 147.4851) (end 107.7087 147.7137) (width 2.2) (layer B.Cu) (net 3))
 (segment (start 106.3498 149.0091) (end 106.3498 147.4851) (width 2.2) (layer B.Cu) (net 3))
 (segment (start 106.3498 147.4851) (end 106.5784 147.7137) (width 2.2) (layer B.Cu) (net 3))
 (segment (start 106.5784 147.7137) (end 107.7087 147.7137) (width 2.2) (layer B.Cu) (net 3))
 (segment (start 107.9881 150.0886) (end 106.3498 151.7269) (width 2.2) (layer B.Cu) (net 3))
 (segment (start 107.7087 147.7137) (end 107.9881 147.9931) (width 2.2) (layer B.Cu) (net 3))
 (segment (start 107.9881 147.9931) (end 107.9881 150.0886) (width 2.2) (layer B.Cu) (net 3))
 (segment (start 106.3498 149.0091) (end 106.3498 151.7269) (width 2.2) (layer B.Cu) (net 3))
 (segment (start 106.3498 151.7269) (end 106.3498 152.4508) (width 2.2) (layer B.Cu) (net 3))
 (segment (start 106.3498 152.4508) (end 107.23372 153.33472) (width 2.2) (layer B.Cu) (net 3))
 (via (at 126.746 153.32964) (size 0.6) (drill 0.4) (layers F.Cu B.Cu) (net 3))
 (segment (start 126.74092 153.33472) (end 126.746 153.32964) (width 2) (layer F.Cu) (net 3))
 (segment (start 126.74092 153.33472) (end 107.23372 153.33472) (width 2) (layer F.Cu) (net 3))
 (via (at 107.23372 153.33472) (size 0.6) (drill 0.4) (layers F.Cu B.Cu) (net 3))
 (segment (start 126.746 152.28824) (end 126.885998 152.148242) (width 2) (layer B.Cu) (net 3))
 (segment (start 126.885998 152.148242) (end 126.885998 151.0284) (width 2) (layer B.Cu) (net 3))
 (segment (start 126.885998 151.0284) (end 126.885998 151.01824) (width 2) (layer B.Cu) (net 3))
 (segment (start 126.885998 151.01824) (end 126.885998 148.1455) (width 2) (layer B.Cu) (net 3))
 (segment (start 126.885998 148.1455) (end 126.746 148.1455) (width 2) (layer B.Cu) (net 3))
 (segment (start 126.785998 148.1455) (end 126.746 148.1455) (width 2.2) (layer B.Cu) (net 3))
 (segment (start 132.3975 159.7914) (end 132.3975 156.7688) (width 2.2) (layer B.Cu) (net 3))
 (segment (start 132.3975 156.7688) (end 131.8641 156.2354) (width 2.2) (layer B.Cu) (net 3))
 (segment (start 131.8641 156.2354) (end 128.5113 156.2354) (width 2.2) (layer B.Cu) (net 3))
 (segment (start 128.5113 156.2354) (end 126.746 154.4701) (width 2.2) (layer B.Cu) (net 3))
 (segment (start 126.746 154.4701) (end 126.746 153.32964) (width 2.2) (layer B.Cu) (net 3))
 (segment (start 126.746 153.32964) (end 126.746 152.28824) (width 2.2) (layer B.Cu) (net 3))
 (segment (start 126.746 150.495) (end 126.746 150.114) (width 2.2) (layer B.Cu) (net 3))
 (segment (start 126.746 150.114) (end 126.746 148.1455) (width 2.2) (layer B.Cu) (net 3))
 (segment (start 126.746 152.28824) (end 126.746 150.495) (width 2.2) (layer B.Cu) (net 3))
 (segment (start 103.8098 149.0091) (end 103.8098 136.264) (width 2) (layer B.Cu) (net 5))
 (segment (start 103.8098 136.264) (end 104.7934 135.2804) (width 2) (layer B.Cu) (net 5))
 (segment (start 106.6419 144.3609) (end 104.267 144.3609) (width 2.2) (layer B.Cu) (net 5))
 (segment (start 104.267 144.3609) (end 103.8479 143.9418) (width 2.2) (layer B.Cu) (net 5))
 (segment (start 142.2273 147.9423) (end 140.2842 147.9423) (width 2.2) (layer B.Cu) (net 5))
 (segment (start 140.2842 147.9423) (end 136.7028 144.3609) (width 2.2) (layer B.Cu) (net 5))
 (segment (start 136.7028 144.3609) (end 106.6419 144.3609) (width 2.2) (layer B.Cu) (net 5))
 (segment (start 103.8479 143.9418) (end 103.8479 141.5669) (width 2) (layer B.Cu) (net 5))
 (segment (start 103.8479 141.5669) (end 103.8479 136.2259) (width 2) (layer B.Cu) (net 5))
 (segment (start 103.8479 136.2259) (end 104.7934 135.2804) (width 2) (layer B.Cu) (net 5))
 (segment (start 135.7376 168.6433) (end 135.7376 169.0878) (width 2) (layer B.Cu) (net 5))
 (segment (start 135.7376 169.0878) (end 135.6741 169.1513) (width 2) (layer B.Cu) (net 5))
 (segment (start 135.6741 169.1513) (end 135.6741 172.7835) (width 2) (layer B.Cu) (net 5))
 (segment (start 138.5824 145.9319) (end 138.5824 146.2405) (width 2) (layer B.Cu) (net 5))
 (segment (start 138.5824 146.2405) (end 140.2842 147.9423) (width 2) (layer B.Cu) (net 5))
 (segment (start 142.2273 147.9423) (end 142.6083 147.9423) (width 2) (layer B.Cu) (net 5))
 (segment (start 103.8479 143.9418) (end 103.8479 157.3911) (width 2) (layer B.Cu) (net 5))
 (segment (start 103.8479 157.3911) (end 101.92512 159.31388) (width 2) (layer B.Cu) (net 5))
 (segment (start 101.92512 159.31388) (end 101.92512 164.62248) (width 2) (layer B.Cu) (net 5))
 (segment (start 101.92512 164.62248) (end 102.35184 165.0492) (width 2) (layer B.Cu) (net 5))
 (segment (start 102.35184 165.0492) (end 104.7369 165.0492) (width 2) (layer B.Cu) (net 5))
 (via (at 121.6152 135.7884) (size 0.6) (drill 0.4) (layers F.Cu B.Cu) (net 5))
 (segment (start 142.6083 136.4361) (end 142.6083 135.8646) (width 2.2) (layer B.Cu) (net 5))
 (via (at 142.6083 135.8646) (size 0.6) (drill 0.4) (layers F.Cu B.Cu) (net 5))
 (segment (start 121.6914 135.8646) (end 142.6083 135.8646) (width 2.2) (layer F.Cu) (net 5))
 (segment (start 121.6914 135.8646) (end 121.6152 135.7884) (width 2.2) (layer F.Cu) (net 5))
 (segment (start 142.6083 136.4361) (end 142.6845 136.4361) (width 2.2) (layer B.Cu) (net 5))
 (segment (start 142.6845 136.4361) (end 142.6083 136.4361) (width 2.2) (layer B.Cu) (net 5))
 (segment (start 142.6083 136.4361) (end 142.6083 137.5791) (width 2.2) (layer B.Cu) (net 5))
 (segment (start 142.6083 137.5791) (end 142.6083 147.9423) (width 2.2) (layer B.Cu) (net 5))
 (segment (start 142.6083 147.9423) (end 142.6083 158.3817) (width 2.2) (layer B.Cu) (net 5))
 (segment (start 140.9446 160.0454) (end 138.8618 160.0454) (width 2.2) (layer B.Cu) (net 5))
 (segment (start 142.6083 158.3817) (end 140.9446 160.0454) (width 2.2) (layer B.Cu) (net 5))
 (segment (start 125.857 127.08) (end 121.6914 127.08) (width 2.2) (layer B.Cu) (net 5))
 (segment (start 122.3391 127.1397) (end 121.6914 127.1397) (width 2.2) (layer B.Cu) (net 5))
 (segment (start 121.7511 127.1397) (end 122.3391 127.1397) (width 2.2) (layer B.Cu) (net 5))
 (segment (start 121.6914 127.08) (end 121.7511 127.1397) (width 2.2) (layer B.Cu) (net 5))
 (segment (start 121.1961 124.54) (end 122.2159 124.54) (width 2.2) (layer B.Cu) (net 5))
 (segment (start 122.2159 124.54) (end 124.7559 127.08) (width 2.2) (layer B.Cu) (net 5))
 (segment (start 125.857 127.08) (end 124.7559 127.08) (width 2.2) (layer B.Cu) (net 5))
 (segment (start 124.7559 127.08) (end 124.1514 127.08) (width 2.2) (layer B.Cu) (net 5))
 (segment (start 124.1514 127.08) (end 121.6914 129.54) (width 2.2) (layer B.Cu) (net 5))
 (segment (start 125.857 127.08) (end 129.667 127.08) (width 2.2) (layer B.Cu) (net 5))
 (segment (start 118.237 124.54) (end 121.1961 124.54) (width 2.2) (layer B.Cu) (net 5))
 (segment (start 121.1961 124.54) (end 121.3777 124.54) (width 2.2) (layer B.Cu) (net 5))
 (segment (start 121.6914 124.8537) (end 121.6914 127.1397) (width 2.2) (layer B.Cu) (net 5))
 (segment (start 121.3777 124.54) (end 121.6914 124.8537) (width 2.2) (layer B.Cu) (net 5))
 (segment (start 121.6914 127.1397) (end 121.6914 129.54) (width 2.2) (layer B.Cu) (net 5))
 (segment (start 118.237 124.54) (end 118.237 121.92) (width 2.2) (layer B.Cu) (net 5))
 (segment (start 118.237 121.92) (end 113.11636 121.92) (width 2.2) (layer B.Cu) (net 5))
 (segment (start 121.6152 135.7884) (end 121.6152 129.6162) (width 2.2) (layer B.Cu) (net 5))
 (segment (start 121.6152 129.6162) (end 121.6914 129.54) (width 2.2) (layer B.Cu) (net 5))
 (segment (start 121.666 137.795) (end 121.666 135.8392) (width 2.2) (layer B.Cu) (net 5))
 (segment (start 121.666 135.8392) (end 121.6152 135.7884) (width 2.2) (layer B.Cu) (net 5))
 (segment (start 121.666 140.5255) (end 121.666 137.795) (width 2.2) (layer B.Cu) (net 5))
 (segment (start 135.6741 168.4782) (end 135.6741 172.7835) (width 2.2) (layer B.Cu) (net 5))
 (segment (start 112.9284 172.72) (end 112.9284 168.6687) (width 2.2) (layer B.Cu) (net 5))
 (segment (start 116.7384 176.53) (end 112.9284 172.72) (width 2.2) (layer B.Cu) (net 5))
 (segment (start 131.9276 176.53) (end 116.7384 176.53) (width 2.2) (layer B.Cu) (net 5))
 (segment (start 135.6741 172.7835) (end 131.9276 176.53) (width 2.2) (layer B.Cu) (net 5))
 (segment (start 104.7369 165.0492) (end 104.7369 168.5163) (width 2.2) (layer B.Cu) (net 5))
 (segment (start 104.8893 168.6687) (end 112.9284 168.6687) (width 2.2) (layer B.Cu) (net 5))
 (segment (start 104.7369 168.5163) (end 104.8893 168.6687) (width 2.2) (layer B.Cu) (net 5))
 (segment (start 112.9284 168.6687) (end 112.9284 165.354) (width 2.2) (layer B.Cu) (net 5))
 (segment (start 135.6741 160.0454) (end 138.8618 160.0454) (width 2.2) (layer B.Cu) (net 5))
 (segment (start 135.6741 168.5925) (end 135.6741 168.4782) (width 2.2) (layer B.Cu) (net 5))
 (segment (start 135.6741 168.4782) (end 135.6741 160.0454) (width 2.2) (layer B.Cu) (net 5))
 (via (at 135.6741 168.5925) (size 0.6) (drill 0.4) (layers F.Cu B.Cu) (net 5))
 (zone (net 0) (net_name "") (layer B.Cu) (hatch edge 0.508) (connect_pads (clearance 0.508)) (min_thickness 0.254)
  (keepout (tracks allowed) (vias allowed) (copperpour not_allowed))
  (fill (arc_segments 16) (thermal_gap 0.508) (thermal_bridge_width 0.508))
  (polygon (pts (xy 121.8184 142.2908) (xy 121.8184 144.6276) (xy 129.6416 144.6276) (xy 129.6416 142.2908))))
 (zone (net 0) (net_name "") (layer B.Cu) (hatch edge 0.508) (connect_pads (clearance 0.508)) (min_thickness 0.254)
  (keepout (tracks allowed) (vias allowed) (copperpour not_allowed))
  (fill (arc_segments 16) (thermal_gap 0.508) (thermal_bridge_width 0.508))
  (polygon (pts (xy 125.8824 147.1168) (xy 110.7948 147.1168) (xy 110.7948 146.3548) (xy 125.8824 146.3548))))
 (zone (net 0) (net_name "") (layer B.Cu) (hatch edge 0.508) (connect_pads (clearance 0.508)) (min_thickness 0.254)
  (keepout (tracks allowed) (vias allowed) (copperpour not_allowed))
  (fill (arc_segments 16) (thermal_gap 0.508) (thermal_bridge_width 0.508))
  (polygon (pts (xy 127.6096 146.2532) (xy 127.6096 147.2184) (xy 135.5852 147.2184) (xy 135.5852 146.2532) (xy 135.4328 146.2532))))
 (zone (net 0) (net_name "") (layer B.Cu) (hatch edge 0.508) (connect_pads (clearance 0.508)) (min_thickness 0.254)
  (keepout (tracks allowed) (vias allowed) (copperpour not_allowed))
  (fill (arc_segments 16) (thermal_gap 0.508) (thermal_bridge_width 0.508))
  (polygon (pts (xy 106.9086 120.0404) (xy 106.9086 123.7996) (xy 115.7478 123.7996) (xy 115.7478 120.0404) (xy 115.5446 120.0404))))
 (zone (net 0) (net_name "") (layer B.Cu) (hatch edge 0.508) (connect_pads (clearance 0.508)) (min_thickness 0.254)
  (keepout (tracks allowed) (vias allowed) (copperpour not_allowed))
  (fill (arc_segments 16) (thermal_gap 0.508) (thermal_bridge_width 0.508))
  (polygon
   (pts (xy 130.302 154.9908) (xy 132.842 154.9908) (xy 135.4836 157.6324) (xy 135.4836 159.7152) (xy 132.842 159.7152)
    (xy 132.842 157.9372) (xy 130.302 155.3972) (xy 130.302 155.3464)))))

